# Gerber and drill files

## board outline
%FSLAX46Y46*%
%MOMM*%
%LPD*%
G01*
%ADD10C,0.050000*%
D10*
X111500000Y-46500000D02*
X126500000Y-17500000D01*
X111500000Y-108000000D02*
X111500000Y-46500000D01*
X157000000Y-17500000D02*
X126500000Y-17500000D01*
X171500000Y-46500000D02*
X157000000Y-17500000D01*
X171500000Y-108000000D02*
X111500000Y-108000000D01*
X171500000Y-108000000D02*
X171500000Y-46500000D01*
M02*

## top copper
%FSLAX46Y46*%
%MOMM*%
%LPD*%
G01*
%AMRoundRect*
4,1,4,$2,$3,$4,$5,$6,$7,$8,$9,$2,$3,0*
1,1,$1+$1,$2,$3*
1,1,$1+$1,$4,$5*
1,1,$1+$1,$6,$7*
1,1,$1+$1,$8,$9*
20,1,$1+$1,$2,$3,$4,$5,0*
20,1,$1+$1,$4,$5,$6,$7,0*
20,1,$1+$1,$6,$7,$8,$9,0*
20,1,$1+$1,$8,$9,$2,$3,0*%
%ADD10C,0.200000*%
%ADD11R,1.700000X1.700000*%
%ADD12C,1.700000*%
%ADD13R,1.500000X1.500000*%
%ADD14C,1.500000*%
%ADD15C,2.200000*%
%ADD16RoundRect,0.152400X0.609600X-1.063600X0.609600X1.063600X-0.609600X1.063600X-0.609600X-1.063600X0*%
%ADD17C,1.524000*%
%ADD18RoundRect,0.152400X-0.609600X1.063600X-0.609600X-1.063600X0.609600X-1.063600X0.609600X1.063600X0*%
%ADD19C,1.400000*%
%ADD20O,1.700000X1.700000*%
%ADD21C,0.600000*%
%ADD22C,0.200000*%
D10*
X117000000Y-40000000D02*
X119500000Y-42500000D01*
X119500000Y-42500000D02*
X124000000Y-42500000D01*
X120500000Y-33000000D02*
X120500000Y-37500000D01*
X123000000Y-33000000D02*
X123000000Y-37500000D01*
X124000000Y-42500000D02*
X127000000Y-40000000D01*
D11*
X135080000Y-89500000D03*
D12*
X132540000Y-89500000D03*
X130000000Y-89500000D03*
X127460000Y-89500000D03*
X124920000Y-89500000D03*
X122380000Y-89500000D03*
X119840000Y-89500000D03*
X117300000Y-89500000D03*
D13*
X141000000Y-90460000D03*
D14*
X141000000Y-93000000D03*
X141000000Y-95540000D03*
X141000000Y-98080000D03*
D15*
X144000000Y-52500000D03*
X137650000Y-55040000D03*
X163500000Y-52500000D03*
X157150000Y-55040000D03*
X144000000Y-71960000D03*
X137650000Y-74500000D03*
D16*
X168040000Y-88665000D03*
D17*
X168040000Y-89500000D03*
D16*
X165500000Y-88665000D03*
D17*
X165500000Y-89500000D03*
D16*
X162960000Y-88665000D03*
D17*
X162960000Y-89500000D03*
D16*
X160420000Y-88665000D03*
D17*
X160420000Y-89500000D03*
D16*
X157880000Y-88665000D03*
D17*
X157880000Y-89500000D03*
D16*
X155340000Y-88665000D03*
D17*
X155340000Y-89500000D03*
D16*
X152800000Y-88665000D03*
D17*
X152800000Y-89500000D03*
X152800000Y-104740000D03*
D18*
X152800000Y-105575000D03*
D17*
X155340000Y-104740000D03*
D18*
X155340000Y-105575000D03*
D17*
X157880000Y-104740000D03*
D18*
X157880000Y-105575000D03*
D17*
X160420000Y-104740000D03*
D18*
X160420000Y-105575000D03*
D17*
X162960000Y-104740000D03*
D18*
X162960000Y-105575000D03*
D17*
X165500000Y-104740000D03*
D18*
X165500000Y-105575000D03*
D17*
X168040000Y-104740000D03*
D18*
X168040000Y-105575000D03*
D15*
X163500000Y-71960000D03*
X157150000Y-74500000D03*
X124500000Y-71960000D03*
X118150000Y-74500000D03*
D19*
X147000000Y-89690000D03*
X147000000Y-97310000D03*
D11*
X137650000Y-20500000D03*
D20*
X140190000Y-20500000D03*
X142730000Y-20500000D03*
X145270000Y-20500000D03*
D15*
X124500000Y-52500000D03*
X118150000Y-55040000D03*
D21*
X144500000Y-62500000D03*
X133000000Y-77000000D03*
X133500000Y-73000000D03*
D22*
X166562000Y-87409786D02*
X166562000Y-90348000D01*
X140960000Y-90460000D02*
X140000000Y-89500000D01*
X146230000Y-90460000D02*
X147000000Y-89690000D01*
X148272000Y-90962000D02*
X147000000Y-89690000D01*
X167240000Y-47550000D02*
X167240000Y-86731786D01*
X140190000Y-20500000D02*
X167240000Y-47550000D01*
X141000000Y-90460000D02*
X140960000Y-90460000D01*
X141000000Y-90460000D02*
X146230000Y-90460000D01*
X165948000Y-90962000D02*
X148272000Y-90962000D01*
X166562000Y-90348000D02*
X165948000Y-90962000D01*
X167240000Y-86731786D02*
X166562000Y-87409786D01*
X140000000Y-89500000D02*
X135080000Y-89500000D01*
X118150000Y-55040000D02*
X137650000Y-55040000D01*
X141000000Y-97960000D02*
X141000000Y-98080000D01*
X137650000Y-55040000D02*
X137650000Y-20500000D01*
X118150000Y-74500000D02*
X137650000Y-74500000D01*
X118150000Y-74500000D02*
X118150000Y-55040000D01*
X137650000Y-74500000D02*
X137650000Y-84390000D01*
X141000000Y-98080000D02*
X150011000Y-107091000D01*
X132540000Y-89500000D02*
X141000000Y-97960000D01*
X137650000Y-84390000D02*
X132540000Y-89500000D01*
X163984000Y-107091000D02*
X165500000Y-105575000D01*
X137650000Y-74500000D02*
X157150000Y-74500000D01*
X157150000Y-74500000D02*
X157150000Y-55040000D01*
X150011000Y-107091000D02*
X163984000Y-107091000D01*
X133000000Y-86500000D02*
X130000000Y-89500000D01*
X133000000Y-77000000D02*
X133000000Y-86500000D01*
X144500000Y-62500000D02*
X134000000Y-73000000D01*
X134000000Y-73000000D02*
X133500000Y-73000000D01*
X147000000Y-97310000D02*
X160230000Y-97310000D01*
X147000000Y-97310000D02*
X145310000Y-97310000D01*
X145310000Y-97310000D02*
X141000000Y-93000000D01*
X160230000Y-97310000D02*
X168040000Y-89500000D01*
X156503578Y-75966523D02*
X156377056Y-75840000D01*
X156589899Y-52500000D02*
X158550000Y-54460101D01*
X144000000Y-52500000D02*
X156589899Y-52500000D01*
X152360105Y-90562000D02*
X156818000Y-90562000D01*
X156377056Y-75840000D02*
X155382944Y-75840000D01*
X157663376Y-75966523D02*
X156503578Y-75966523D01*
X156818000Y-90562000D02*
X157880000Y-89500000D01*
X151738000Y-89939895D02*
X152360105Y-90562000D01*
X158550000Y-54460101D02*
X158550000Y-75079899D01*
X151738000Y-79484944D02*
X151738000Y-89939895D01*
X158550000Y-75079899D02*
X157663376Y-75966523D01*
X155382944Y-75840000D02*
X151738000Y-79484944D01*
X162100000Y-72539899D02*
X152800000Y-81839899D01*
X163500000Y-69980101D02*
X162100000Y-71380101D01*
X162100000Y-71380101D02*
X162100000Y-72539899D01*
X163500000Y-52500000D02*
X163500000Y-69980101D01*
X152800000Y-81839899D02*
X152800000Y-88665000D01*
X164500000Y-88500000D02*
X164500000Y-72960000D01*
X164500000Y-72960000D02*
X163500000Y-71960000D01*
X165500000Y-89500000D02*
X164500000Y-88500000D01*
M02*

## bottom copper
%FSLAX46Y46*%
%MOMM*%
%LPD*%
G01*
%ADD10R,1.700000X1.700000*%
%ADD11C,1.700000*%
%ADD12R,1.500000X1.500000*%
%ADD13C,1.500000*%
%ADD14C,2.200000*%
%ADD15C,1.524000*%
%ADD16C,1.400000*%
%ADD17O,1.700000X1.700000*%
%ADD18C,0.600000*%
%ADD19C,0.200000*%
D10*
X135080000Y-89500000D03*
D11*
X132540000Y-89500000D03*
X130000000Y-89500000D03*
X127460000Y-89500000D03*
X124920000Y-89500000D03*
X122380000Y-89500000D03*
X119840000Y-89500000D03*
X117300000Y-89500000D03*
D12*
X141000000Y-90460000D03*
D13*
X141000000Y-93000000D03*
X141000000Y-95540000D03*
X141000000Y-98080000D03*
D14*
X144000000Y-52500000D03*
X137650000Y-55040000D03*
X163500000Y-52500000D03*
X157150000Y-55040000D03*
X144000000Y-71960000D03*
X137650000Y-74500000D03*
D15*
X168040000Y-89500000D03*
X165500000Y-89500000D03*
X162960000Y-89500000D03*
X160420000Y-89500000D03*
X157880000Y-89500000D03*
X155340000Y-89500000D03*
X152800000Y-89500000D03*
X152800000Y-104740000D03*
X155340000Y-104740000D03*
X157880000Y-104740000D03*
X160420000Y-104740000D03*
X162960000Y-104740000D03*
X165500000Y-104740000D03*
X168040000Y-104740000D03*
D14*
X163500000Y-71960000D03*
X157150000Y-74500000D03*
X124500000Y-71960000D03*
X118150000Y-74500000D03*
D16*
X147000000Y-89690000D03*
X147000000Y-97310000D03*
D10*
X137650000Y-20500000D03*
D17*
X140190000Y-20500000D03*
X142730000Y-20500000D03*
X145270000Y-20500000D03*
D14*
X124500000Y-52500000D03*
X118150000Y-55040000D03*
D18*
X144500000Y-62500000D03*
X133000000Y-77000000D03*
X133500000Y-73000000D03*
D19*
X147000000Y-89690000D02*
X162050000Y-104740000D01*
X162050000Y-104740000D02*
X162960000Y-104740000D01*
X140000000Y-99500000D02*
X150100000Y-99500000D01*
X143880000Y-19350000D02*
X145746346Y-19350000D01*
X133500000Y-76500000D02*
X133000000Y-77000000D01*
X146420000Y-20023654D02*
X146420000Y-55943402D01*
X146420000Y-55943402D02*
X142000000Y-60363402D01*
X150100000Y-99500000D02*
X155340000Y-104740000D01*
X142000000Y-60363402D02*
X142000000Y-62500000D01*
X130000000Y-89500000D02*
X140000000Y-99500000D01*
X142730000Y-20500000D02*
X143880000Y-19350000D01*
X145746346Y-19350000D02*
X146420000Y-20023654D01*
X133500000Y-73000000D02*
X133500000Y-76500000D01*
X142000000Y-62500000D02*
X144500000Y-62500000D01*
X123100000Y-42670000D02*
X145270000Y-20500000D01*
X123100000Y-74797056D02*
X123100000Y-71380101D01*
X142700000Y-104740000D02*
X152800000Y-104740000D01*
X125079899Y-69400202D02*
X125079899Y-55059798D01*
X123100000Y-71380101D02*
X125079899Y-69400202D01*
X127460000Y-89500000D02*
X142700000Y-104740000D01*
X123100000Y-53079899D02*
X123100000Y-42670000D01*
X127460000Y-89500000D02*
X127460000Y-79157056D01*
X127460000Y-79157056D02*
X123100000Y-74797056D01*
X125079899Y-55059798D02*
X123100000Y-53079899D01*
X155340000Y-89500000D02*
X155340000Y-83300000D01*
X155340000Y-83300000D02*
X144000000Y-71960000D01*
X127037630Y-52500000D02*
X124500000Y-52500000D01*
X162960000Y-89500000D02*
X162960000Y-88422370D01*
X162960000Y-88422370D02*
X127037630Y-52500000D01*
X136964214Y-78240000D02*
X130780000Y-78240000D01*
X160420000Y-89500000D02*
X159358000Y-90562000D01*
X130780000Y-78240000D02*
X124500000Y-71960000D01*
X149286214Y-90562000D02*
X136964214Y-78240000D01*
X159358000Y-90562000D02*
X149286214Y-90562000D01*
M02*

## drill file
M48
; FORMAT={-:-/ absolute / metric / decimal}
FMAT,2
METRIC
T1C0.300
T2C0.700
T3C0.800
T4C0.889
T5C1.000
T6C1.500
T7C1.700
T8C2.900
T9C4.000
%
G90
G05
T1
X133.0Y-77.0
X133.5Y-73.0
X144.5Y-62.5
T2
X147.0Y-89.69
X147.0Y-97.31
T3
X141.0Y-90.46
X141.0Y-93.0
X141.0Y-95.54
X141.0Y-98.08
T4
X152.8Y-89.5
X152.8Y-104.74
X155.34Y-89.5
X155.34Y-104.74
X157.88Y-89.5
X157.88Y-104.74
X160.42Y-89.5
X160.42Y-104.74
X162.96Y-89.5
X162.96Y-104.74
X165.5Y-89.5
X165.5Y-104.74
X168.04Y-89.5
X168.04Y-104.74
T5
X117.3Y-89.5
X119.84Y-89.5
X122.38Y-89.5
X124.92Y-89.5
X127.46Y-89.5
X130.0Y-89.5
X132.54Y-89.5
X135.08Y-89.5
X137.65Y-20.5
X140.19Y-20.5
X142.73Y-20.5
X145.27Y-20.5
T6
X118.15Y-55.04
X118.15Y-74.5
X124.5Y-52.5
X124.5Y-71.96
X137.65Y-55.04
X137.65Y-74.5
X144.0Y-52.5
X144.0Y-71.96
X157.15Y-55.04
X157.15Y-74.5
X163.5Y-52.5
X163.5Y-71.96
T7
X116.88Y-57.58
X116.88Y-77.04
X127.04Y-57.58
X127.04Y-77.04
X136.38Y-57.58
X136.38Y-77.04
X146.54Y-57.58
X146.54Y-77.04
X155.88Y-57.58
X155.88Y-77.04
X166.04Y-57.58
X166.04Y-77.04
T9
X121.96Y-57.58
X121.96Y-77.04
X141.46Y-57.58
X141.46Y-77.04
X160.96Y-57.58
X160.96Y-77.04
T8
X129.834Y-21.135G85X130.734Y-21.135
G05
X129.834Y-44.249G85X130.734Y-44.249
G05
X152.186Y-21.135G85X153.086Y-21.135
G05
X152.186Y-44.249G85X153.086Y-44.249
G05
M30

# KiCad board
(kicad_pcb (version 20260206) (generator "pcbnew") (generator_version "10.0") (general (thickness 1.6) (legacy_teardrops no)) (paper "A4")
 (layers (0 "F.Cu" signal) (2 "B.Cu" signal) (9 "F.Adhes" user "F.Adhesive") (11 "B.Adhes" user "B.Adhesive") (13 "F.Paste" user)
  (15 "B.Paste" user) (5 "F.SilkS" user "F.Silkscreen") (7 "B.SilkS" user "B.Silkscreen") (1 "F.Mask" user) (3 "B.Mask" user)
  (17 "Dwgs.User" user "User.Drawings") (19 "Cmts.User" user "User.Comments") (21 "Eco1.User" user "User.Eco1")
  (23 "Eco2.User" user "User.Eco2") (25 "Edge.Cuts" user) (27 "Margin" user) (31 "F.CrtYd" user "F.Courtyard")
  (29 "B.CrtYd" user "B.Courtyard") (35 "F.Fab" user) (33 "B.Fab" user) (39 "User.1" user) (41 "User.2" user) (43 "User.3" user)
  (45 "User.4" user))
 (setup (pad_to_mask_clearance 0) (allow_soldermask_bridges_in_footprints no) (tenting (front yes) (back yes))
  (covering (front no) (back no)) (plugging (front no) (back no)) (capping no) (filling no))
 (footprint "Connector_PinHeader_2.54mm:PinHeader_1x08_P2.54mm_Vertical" (layer "F.Cu") (at 135.08 89.5 -90)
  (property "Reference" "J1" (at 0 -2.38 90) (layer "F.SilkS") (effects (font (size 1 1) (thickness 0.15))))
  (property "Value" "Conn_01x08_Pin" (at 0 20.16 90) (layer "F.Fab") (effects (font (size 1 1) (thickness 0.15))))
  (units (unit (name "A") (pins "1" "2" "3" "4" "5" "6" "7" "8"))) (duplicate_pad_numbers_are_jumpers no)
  (pad "1" thru_hole rect (at 0 0 270) (size 1.7 1.7) (drill 1) (layers "*.Cu" "*.Mask") (remove_unused_layers no) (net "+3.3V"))
  (pad "2" thru_hole circle (at 0 2.54 270) (size 1.7 1.7) (drill 1) (layers "*.Cu" "*.Mask") (remove_unused_layers no) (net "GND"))
  (pad "3" thru_hole circle (at 0 5.08 270) (size 1.7 1.7) (drill 1) (layers "*.Cu" "*.Mask") (remove_unused_layers no) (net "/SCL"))
  (pad "4" thru_hole circle (at 0 7.62 270) (size 1.7 1.7) (drill 1) (layers "*.Cu" "*.Mask") (remove_unused_layers no) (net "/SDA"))
  (pad "5" thru_hole circle (at 0 10.16 270) (size 1.7 1.7) (drill 1) (layers "*.Cu" "*.Mask") (remove_unused_layers no)
   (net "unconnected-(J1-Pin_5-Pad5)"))
  (pad "6" thru_hole circle (at 0 12.7 270) (size 1.7 1.7) (drill 1) (layers "*.Cu" "*.Mask") (remove_unused_layers no)
   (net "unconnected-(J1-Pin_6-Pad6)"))
  (pad "7" thru_hole circle (at 0 15.24 270) (size 1.7 1.7) (drill 1) (layers "*.Cu" "*.Mask") (remove_unused_layers no)
   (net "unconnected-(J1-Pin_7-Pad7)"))
  (pad "8" thru_hole circle (at 0 17.78 270) (size 1.7 1.7) (drill 1) (layers "*.Cu" "*.Mask") (remove_unused_layers no)
   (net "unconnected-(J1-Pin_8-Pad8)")))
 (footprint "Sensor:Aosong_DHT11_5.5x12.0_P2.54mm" (layer "F.Cu") (at 141 90.46)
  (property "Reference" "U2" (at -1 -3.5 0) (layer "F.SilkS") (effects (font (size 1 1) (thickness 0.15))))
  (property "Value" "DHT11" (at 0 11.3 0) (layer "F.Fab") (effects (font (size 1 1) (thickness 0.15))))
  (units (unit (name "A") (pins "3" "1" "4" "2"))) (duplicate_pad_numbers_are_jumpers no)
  (pad "1" thru_hole rect (at 0 0) (size 1.5 1.5) (drill 0.8) (layers "*.Cu" "*.Mask") (remove_unused_layers no) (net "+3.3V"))
  (pad "2" thru_hole circle (at 0 2.54) (size 1.5 1.5) (drill 0.8) (layers "*.Cu" "*.Mask") (remove_unused_layers no) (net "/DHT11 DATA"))
  (pad "3" thru_hole circle (at 0 5.08) (size 1.5 1.5) (drill 0.8) (layers "*.Cu" "*.Mask") (remove_unused_layers no)
   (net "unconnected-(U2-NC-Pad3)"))
  (pad "4" thru_hole circle (at 0 7.62) (size 1.5 1.5) (drill 0.8) (layers "*.Cu" "*.Mask") (remove_unused_layers no) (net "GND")))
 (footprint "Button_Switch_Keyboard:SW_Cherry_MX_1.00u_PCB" (layer "F.Cu") (at 144 52.5)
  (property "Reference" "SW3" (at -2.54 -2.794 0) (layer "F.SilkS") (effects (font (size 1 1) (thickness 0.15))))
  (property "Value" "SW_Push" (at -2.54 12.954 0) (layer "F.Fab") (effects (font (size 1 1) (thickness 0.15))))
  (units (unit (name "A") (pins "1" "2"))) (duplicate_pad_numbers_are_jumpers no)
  (pad "" np_thru_hole circle (at -7.62 5.08) (size 1.7 1.7) (drill 1.7) (layers "*.Cu" "*.Mask"))
  (pad "" np_thru_hole circle (at -2.54 5.08) (size 4 4) (drill 4) (layers "*.Cu" "*.Mask"))
  (pad "" np_thru_hole circle (at 2.54 5.08) (size 1.7 1.7) (drill 1.7) (layers "*.Cu" "*.Mask"))
  (pad "1" thru_hole circle (at 0 0) (size 2.2 2.2) (drill 1.5) (layers "*.Cu" "*.Mask") (remove_unused_layers no) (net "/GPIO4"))
  (pad "2" thru_hole circle (at -6.35 2.54) (size 2.2 2.2) (drill 1.5) (layers "*.Cu" "*.Mask") (remove_unused_layers no) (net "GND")))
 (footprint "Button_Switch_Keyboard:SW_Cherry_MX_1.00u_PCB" (layer "F.Cu") (at 163.5 52.5)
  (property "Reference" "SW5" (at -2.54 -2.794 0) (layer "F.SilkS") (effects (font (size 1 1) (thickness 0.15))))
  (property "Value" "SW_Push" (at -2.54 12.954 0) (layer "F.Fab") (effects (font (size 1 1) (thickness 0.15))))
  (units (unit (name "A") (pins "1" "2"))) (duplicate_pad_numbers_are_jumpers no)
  (pad "" np_thru_hole circle (at -7.62 5.08) (size 1.7 1.7) (drill 1.7) (layers "*.Cu" "*.Mask"))
  (pad "" np_thru_hole circle (at -2.54 5.08) (size 4 4) (drill 4) (layers "*.Cu" "*.Mask"))
  (pad "" np_thru_hole circle (at 2.54 5.08) (size 1.7 1.7) (drill 1.7) (layers "*.Cu" "*.Mask"))
  (pad "1" thru_hole circle (at 0 0) (size 2.2 2.2) (drill 1.5) (layers "*.Cu" "*.Mask") (remove_unused_layers no) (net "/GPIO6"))
  (pad "2" thru_hole circle (at -6.35 2.54) (size 2.2 2.2) (drill 1.5) (layers "*.Cu" "*.Mask") (remove_unused_layers no) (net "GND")))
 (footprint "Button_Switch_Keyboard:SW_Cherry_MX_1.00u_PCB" (layer "F.Cu") (at 144 71.96)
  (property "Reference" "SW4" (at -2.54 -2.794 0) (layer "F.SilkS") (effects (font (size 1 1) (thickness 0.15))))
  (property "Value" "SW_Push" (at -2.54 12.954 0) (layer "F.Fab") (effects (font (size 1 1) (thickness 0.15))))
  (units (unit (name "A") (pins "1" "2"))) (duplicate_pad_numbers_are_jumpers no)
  (pad "" np_thru_hole circle (at -7.62 5.08) (size 1.7 1.7) (drill 1.7) (layers "*.Cu" "*.Mask"))
  (pad "" np_thru_hole circle (at -2.54 5.08) (size 4 4) (drill 4) (layers "*.Cu" "*.Mask"))
  (pad "" np_thru_hole circle (at 2.54 5.08) (size 1.7 1.7) (drill 1.7) (layers "*.Cu" "*.Mask"))
  (pad "1" thru_hole circle (at 0 0) (size 2.2 2.2) (drill 1.5) (layers "*.Cu" "*.Mask") (remove_unused_layers no) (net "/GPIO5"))
  (pad "2" thru_hole circle (at -6.35 2.54) (size 2.2 2.2) (drill 1.5) (layers "*.Cu" "*.Mask") (remove_unused_layers no) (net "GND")))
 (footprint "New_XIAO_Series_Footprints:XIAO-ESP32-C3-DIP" (layer "F.Cu") (at 160.42 97.12)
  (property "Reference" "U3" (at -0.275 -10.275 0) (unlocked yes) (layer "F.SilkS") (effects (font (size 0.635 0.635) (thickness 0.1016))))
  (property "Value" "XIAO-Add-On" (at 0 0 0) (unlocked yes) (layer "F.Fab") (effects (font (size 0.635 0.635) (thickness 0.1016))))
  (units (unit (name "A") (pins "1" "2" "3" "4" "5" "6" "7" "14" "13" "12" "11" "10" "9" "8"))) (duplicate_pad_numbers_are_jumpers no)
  (pad "1" smd roundrect (at 7.62 -8.455 90) (size 2.432 1.524) (layers "F.Cu" "F.Mask") (roundrect_rratio 0.1) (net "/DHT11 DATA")
   (thermal_bridge_angle 45))
  (pad "1" thru_hole circle (at 7.62 -7.62 90) (size 1.524 1.524) (drill 0.889) (layers "*.Cu" "*.Mask") (remove_unused_layers no)
   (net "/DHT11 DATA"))
  (pad "2" smd roundrect (at 5.08 -8.455 90) (size 2.432 1.524) (layers "F.Cu" "F.Mask") (roundrect_rratio 0.1) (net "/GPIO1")
   (thermal_bridge_angle 45))
  (pad "2" thru_hole circle (at 5.08 -7.62 90) (size 1.524 1.524) (drill 0.889) (layers "*.Cu" "*.Mask") (remove_unused_layers no)
   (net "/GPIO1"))
  (pad "3" smd roundrect (at 2.54 -8.455 90) (size 2.432 1.524) (layers "F.Cu" "F.Mask") (roundrect_rratio 0.1) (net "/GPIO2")
   (thermal_bridge_angle 45))
  (pad "3" thru_hole circle (at 2.54 -7.62 90) (size 1.524 1.524) (drill 0.889) (layers "*.Cu" "*.Mask") (remove_unused_layers no)
   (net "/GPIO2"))
  (pad "4" smd roundrect (at 0 -8.455 90) (size 2.432 1.524) (layers "F.Cu" "F.Mask") (roundrect_rratio 0.1) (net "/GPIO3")
   (thermal_bridge_angle 45))
  (pad "4" thru_hole circle (at 0 -7.62 90) (size 1.524 1.524) (drill 0.889) (layers "*.Cu" "*.Mask") (remove_unused_layers no)
   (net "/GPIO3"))
  (pad "5" smd roundrect (at -2.54 -8.455 90) (size 2.432 1.524) (layers "F.Cu" "F.Mask") (roundrect_rratio 0.1) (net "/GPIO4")
   (thermal_bridge_angle 45))
  (pad "5" thru_hole circle (at -2.54 -7.62 90) (size 1.524 1.524) (drill 0.889) (layers "*.Cu" "*.Mask") (remove_unused_layers no)
   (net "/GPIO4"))
  (pad "6" smd roundrect (at -5.08 -8.455 90) (size 2.432 1.524) (layers "F.Cu" "F.Mask") (roundrect_rratio 0.1) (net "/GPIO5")
   (thermal_bridge_angle 45))
  (pad "6" thru_hole circle (at -5.08 -7.62 90) (size 1.524 1.524) (drill 0.889) (layers "*.Cu" "*.Mask") (remove_unused_layers no)
   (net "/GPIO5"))
  (pad "7" smd roundrect (at -7.62 -8.455 90) (size 2.432 1.524) (layers "F.Cu" "F.Mask") (roundrect_rratio 0.1) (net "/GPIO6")
   (thermal_bridge_angle 45))
  (pad "7" thru_hole circle (at -7.62 -7.62 90) (size 1.524 1.524) (drill 0.889) (layers "*.Cu" "*.Mask") (remove_unused_layers no)
   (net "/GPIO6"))
  (pad "8" thru_hole circle (at -7.62 7.62 270) (size 1.524 1.524) (drill 0.889) (layers "*.Cu" "*.Mask") (remove_unused_layers no)
   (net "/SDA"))
  (pad "8" smd roundrect (at -7.62 8.455 270) (size 2.432 1.524) (layers "F.Cu" "F.Mask") (roundrect_rratio 0.1) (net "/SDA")
   (thermal_bridge_angle 45))
  (pad "9" thru_hole circle (at -5.08 7.62 270) (size 1.524 1.524) (drill 0.889) (layers "*.Cu" "*.Mask") (remove_unused_layers no)
   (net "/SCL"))
  (pad "9" smd roundrect (at -5.08 8.455 270) (size 2.432 1.524) (layers "F.Cu" "F.Mask") (roundrect_rratio 0.1) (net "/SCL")
   (thermal_bridge_angle 45))
  (pad "10" thru_hole circle (at -2.54 7.62 270) (size 1.524 1.524) (drill 0.889) (layers "*.Cu" "*.Mask") (remove_unused_layers no)
   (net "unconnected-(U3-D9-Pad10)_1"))
  (pad "10" smd roundrect (at -2.54 8.455 270) (size 2.432 1.524) (layers "F.Cu" "F.Mask") (roundrect_rratio 0.1)
   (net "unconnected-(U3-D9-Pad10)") (thermal_bridge_angle 45))
  (pad "11" thru_hole circle (at 0 7.62 270) (size 1.524 1.524) (drill 0.889) (layers "*.Cu" "*.Mask") (remove_unused_layers no)
   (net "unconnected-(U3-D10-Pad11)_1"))
  (pad "11" smd roundrect (at 0 8.455 270) (size 2.432 1.524) (layers "F.Cu" "F.Mask") (roundrect_rratio 0.1)
   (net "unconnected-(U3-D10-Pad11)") (thermal_bridge_angle 45))
  (pad "12" thru_hole circle (at 2.54 7.62 270) (size 1.524 1.524) (drill 0.889) (layers "*.Cu" "*.Mask") (remove_unused_layers no)
   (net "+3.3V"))
  (pad "12" smd roundrect (at 2.54 8.455 270) (size 2.432 1.524) (layers "F.Cu" "F.Mask") (roundrect_rratio 0.1) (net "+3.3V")
   (thermal_bridge_angle 45))
  (pad "13" thru_hole circle (at 5.08 7.62 270) (size 1.524 1.524) (drill 0.889) (layers "*.Cu" "*.Mask") (remove_unused_layers no)
   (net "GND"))
  (pad "13" smd roundrect (at 5.08 8.455 270) (size 2.432 1.524) (layers "F.Cu" "F.Mask") (roundrect_rratio 0.1) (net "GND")
   (thermal_bridge_angle 45))
  (pad "14" thru_hole circle (at 7.62 7.62 270) (size 1.524 1.524) (drill 0.889) (layers "*.Cu" "*.Mask") (remove_unused_layers no)
   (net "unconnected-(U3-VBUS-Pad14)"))
  (pad "14" smd roundrect (at 7.62 8.455 270) (size 2.432 1.524) (layers "F.Cu" "F.Mask") (roundrect_rratio 0.1)
   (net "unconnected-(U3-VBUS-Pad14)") (thermal_bridge_angle 45)))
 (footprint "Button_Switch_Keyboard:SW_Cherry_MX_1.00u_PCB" (layer "F.Cu") (at 163.5 71.96)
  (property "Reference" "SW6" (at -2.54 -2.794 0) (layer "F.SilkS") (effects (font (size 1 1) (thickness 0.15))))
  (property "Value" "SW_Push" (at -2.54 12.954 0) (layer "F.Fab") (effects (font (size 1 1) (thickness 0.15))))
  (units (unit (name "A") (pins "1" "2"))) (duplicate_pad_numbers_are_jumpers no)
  (pad "" np_thru_hole circle (at -7.62 5.08) (size 1.7 1.7) (drill 1.7) (layers "*.Cu" "*.Mask"))
  (pad "" np_thru_hole circle (at -2.54 5.08) (size 4 4) (drill 4) (layers "*.Cu" "*.Mask"))
  (pad "" np_thru_hole circle (at 2.54 5.08) (size 1.7 1.7) (drill 1.7) (layers "*.Cu" "*.Mask"))
  (pad "1" thru_hole circle (at 0 0) (size 2.2 2.2) (drill 1.5) (layers "*.Cu" "*.Mask") (remove_unused_layers no) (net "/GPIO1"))
  (pad "2" thru_hole circle (at -6.35 2.54) (size 2.2 2.2) (drill 1.5) (layers "*.Cu" "*.Mask") (remove_unused_layers no) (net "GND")))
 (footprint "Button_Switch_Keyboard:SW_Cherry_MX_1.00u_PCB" (layer "F.Cu") (at 124.5 71.96)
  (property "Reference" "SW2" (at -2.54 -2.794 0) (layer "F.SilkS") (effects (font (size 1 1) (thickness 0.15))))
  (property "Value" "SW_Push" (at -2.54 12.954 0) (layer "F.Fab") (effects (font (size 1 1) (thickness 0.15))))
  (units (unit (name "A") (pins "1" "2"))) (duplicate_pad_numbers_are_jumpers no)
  (pad "" np_thru_hole circle (at -7.62 5.08) (size 1.7 1.7) (drill 1.7) (layers "*.Cu" "*.Mask"))
  (pad "" np_thru_hole circle (at -2.54 5.08) (size 4 4) (drill 4) (layers "*.Cu" "*.Mask"))
  (pad "" np_thru_hole circle (at 2.54 5.08) (size 1.7 1.7) (drill 1.7) (layers "*.Cu" "*.Mask"))
  (pad "1" thru_hole circle (at 0 0) (size 2.2 2.2) (drill 1.5) (layers "*.Cu" "*.Mask") (remove_unused_layers no) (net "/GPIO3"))
  (pad "2" thru_hole circle (at -6.35 2.54) (size 2.2 2.2) (drill 1.5) (layers "*.Cu" "*.Mask") (remove_unused_layers no) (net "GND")))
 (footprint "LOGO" (layer "F.Cu") (at 161.5 39.5)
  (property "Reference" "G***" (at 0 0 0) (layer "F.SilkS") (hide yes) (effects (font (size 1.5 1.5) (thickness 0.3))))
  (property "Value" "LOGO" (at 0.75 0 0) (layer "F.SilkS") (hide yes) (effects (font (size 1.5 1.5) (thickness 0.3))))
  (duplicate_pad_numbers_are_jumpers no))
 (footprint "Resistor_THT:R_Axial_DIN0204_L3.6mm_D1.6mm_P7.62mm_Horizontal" (layer "F.Cu") (at 147 89.69 -90)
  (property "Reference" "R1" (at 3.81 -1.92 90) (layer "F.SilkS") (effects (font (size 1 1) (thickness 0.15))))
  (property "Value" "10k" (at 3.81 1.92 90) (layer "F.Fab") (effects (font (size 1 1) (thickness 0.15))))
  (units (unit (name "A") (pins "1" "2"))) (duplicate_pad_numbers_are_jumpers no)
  (pad "1" thru_hole circle (at 0 0 270) (size 1.4 1.4) (drill 0.7) (layers "*.Cu" "*.Mask") (remove_unused_layers no) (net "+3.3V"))
  (pad "2" thru_hole circle (at 7.62 0 270) (size 1.4 1.4) (drill 0.7) (layers "*.Cu" "*.Mask") (remove_unused_layers no)
   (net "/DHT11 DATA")))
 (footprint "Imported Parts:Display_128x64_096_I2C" (layer "F.Cu") (at 141.46 20.5)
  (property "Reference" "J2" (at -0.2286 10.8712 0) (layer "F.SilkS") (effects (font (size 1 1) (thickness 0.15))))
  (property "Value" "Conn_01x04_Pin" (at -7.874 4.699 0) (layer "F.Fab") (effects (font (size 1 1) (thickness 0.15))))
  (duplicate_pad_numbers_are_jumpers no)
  (pad "" np_thru_hole oval (at -11.176 0.635) (size 3.8 2.9) (drill oval 3.8 2.9) (layers "*.Cu" "*.Mask"))
  (pad "" np_thru_hole oval (at -11.176 23.749) (size 3.8 2.9) (drill oval 3.8 2.9) (layers "*.Cu" "*.Mask"))
  (pad "" np_thru_hole oval (at 11.176 0.635) (size 3.8 2.9) (drill oval 3.8 2.9) (layers "*.Cu" "*.Mask"))
  (pad "" np_thru_hole oval (at 11.176 23.749) (size 3.8 2.9) (drill oval 3.8 2.9) (layers "*.Cu" "*.Mask"))
  (pad "1" thru_hole rect (at -3.81 0 90) (size 1.7 1.7) (drill 1) (layers "*.Cu" "*.Mask") (remove_unused_layers no) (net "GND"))
  (pad "2" thru_hole oval (at -1.27 0 90) (size 1.7 1.7) (drill 1) (layers "*.Cu" "*.Mask") (remove_unused_layers no) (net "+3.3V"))
  (pad "3" thru_hole oval (at 1.27 0 90) (size 1.7 1.7) (drill 1) (layers "*.Cu" "*.Mask") (remove_unused_layers no) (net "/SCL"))
  (pad "4" thru_hole oval (at 3.81 0 90) (size 1.7 1.7) (drill 1) (layers "*.Cu" "*.Mask") (remove_unused_layers no) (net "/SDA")))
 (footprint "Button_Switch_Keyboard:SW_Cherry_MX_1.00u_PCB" (layer "F.Cu") (at 124.5 52.5)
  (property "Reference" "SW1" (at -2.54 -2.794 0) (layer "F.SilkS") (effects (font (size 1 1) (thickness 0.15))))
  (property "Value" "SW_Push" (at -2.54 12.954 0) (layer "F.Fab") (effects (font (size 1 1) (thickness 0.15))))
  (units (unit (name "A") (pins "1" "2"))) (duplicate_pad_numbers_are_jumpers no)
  (pad "" np_thru_hole circle (at -7.62 5.08) (size 1.7 1.7) (drill 1.7) (layers "*.Cu" "*.Mask"))
  (pad "" np_thru_hole circle (at -2.54 5.08) (size 4 4) (drill 4) (layers "*.Cu" "*.Mask"))
  (pad "" np_thru_hole circle (at 2.54 5.08) (size 1.7 1.7) (drill 1.7) (layers "*.Cu" "*.Mask"))
  (pad "1" thru_hole circle (at 0 0) (size 2.2 2.2) (drill 1.5) (layers "*.Cu" "*.Mask") (remove_unused_layers no) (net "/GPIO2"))
  (pad "2" thru_hole circle (at -6.35 2.54) (size 2.2 2.2) (drill 1.5) (layers "*.Cu" "*.Mask") (remove_unused_layers no) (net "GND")))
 (gr_line (start 117 40) (end 119.5 42.5) (stroke (width 0.2) (type default)) (layer "F.Cu"))
 (gr_line (start 119.5 42.5) (end 124 42.5) (stroke (width 0.2) (type default)) (layer "F.Cu"))
 (gr_line (start 120.5 33) (end 120.5 37.5) (stroke (width 0.2) (type default)) (layer "F.Cu"))
 (gr_line (start 123 33) (end 123 37.5) (stroke (width 0.2) (type default)) (layer "F.Cu"))
 (gr_line (start 124 42.5) (end 127 40) (stroke (width 0.2) (type default)) (layer "F.Cu"))
 (gr_line (start 111.5 46.5) (end 126.5 17.5) (stroke (width 0.05) (type default)) (layer "Edge.Cuts"))
 (gr_line (start 111.5 108) (end 111.5 46.5) (stroke (width 0.05) (type default)) (layer "Edge.Cuts"))
 (gr_line (start 157 17.5) (end 126.5 17.5) (stroke (width 0.05) (type default)) (layer "Edge.Cuts"))
 (gr_line (start 171.5 46.5) (end 157 17.5) (stroke (width 0.05) (type default)) (layer "Edge.Cuts"))
 (gr_line (start 171.5 108) (end 111.5 108) (stroke (width 0.05) (type default)) (layer "Edge.Cuts"))
 (gr_line (start 171.5 108) (end 171.5 46.5) (stroke (width 0.05) (type default)) (layer "Edge.Cuts"))
 (segment (start 166.562 87.409786) (end 166.562 90.348) (width 0.2) (layer "F.Cu") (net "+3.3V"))
 (segment (start 140.96 90.46) (end 140 89.5) (width 0.2) (layer "F.Cu") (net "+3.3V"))
 (segment (start 146.23 90.46) (end 147 89.69) (width 0.2) (layer "F.Cu") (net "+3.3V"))
 (segment (start 148.272 90.962) (end 147 89.69) (width 0.2) (layer "F.Cu") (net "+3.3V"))
 (segment (start 167.24 47.55) (end 167.24 86.731786) (width 0.2) (layer "F.Cu") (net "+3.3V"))
 (segment (start 140.19 20.5) (end 167.24 47.55) (width 0.2) (layer "F.Cu") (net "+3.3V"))
 (segment (start 141 90.46) (end 140.96 90.46) (width 0.2) (layer "F.Cu") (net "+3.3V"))
 (segment (start 141 90.46) (end 146.23 90.46) (width 0.2) (layer "F.Cu") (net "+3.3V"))
 (segment (start 165.948 90.962) (end 148.272 90.962) (width 0.2) (layer "F.Cu") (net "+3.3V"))
 (segment (start 166.562 90.348) (end 165.948 90.962) (width 0.2) (layer "F.Cu") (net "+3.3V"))
 (segment (start 167.24 86.731786) (end 166.562 87.409786) (width 0.2) (layer "F.Cu") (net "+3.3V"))
 (segment (start 140 89.5) (end 135.08 89.5) (width 0.2) (layer "F.Cu") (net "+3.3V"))
 (segment (start 147 89.69) (end 162.05 104.74) (width 0.2) (layer "B.Cu") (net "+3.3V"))
 (segment (start 162.05 104.74) (end 162.96 104.74) (width 0.2) (layer "B.Cu") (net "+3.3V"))
 (segment (start 118.15 55.04) (end 137.65 55.04) (width 0.2) (layer "F.Cu") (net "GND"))
 (segment (start 141 97.96) (end 141 98.08) (width 0.2) (layer "F.Cu") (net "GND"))
 (segment (start 137.65 55.04) (end 137.65 20.5) (width 0.2) (layer "F.Cu") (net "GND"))
 (segment (start 118.15 74.5) (end 137.65 74.5) (width 0.2) (layer "F.Cu") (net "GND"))
 (segment (start 118.15 74.5) (end 118.15 55.04) (width 0.2) (layer "F.Cu") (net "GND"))
 (segment (start 137.65 74.5) (end 137.65 84.39) (width 0.2) (layer "F.Cu") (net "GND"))
 (segment (start 141 98.08) (end 150.011 107.091) (width 0.2) (layer "F.Cu") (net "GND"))
 (segment (start 132.54 89.5) (end 141 97.96) (width 0.2) (layer "F.Cu") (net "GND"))
 (segment (start 137.65 84.39) (end 132.54 89.5) (width 0.2) (layer "F.Cu") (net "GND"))
 (segment (start 163.984 107.091) (end 165.5 105.575) (width 0.2) (layer "F.Cu") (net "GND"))
 (segment (start 137.65 74.5) (end 157.15 74.5) (width 0.2) (layer "F.Cu") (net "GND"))
 (segment (start 157.15 74.5) (end 157.15 55.04) (width 0.2) (layer "F.Cu") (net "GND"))
 (segment (start 150.011 107.091) (end 163.984 107.091) (width 0.2) (layer "F.Cu") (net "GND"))
 (segment (start 133 86.5) (end 130 89.5) (width 0.2) (layer "F.Cu") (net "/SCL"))
 (segment (start 133 77) (end 133 86.5) (width 0.2) (layer "F.Cu") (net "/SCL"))
 (segment (start 144.5 62.5) (end 134 73) (width 0.2) (layer "F.Cu") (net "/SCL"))
 (segment (start 134 73) (end 133.5 73) (width 0.2) (layer "F.Cu") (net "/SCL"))
 (via (at 144.5 62.5) (size 0.6) (drill 0.3) (layers "F.Cu" "B.Cu") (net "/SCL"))
 (via (at 133 77) (size 0.6) (drill 0.3) (layers "F.Cu" "B.Cu") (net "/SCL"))
 (via (at 133.5 73) (size 0.6) (drill 0.3) (layers "F.Cu" "B.Cu") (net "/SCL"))
 (segment (start 140 99.5) (end 150.1 99.5) (width 0.2) (layer "B.Cu") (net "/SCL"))
 (segment (start 143.88 19.35) (end 145.746346 19.35) (width 0.2) (layer "B.Cu") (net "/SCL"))
 (segment (start 133.5 76.5) (end 133 77) (width 0.2) (layer "B.Cu") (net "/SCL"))
 (segment (start 146.42 20.023654) (end 146.42 55.943402) (width 0.2) (layer "B.Cu") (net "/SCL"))
 (segment (start 146.42 55.943402) (end 142 60.363402) (width 0.2) (layer "B.Cu") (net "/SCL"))
 (segment (start 150.1 99.5) (end 155.34 104.74) (width 0.2) (layer "B.Cu") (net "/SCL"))
 (segment (start 142 60.363402) (end 142 62.5) (width 0.2) (layer "B.Cu") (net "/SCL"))
 (segment (start 130 89.5) (end 140 99.5) (width 0.2) (layer "B.Cu") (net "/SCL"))
 (segment (start 142.73 20.5) (end 143.88 19.35) (width 0.2) (layer "B.Cu") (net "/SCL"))
 (segment (start 145.746346 19.35) (end 146.42 20.023654) (width 0.2) (layer "B.Cu") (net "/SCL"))
 (segment (start 133.5 73) (end 133.5 76.5) (width 0.2) (layer "B.Cu") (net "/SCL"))
 (segment (start 142 62.5) (end 144.5 62.5) (width 0.2) (layer "B.Cu") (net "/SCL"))
 (segment (start 123.1 42.67) (end 145.27 20.5) (width 0.2) (layer "B.Cu") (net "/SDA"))
 (segment (start 123.1 74.797056) (end 123.1 71.380101) (width 0.2) (layer "B.Cu") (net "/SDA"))
 (segment (start 142.7 104.74) (end 152.8 104.74) (width 0.2) (layer "B.Cu") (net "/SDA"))
 (segment (start 125.079899 69.400202) (end 125.079899 55.059798) (width 0.2) (layer "B.Cu") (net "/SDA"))
 (segment (start 123.1 71.380101) (end 125.079899 69.400202) (width 0.2) (layer "B.Cu") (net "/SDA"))
 (segment (start 127.46 89.5) (end 142.7 104.74) (width 0.2) (layer "B.Cu") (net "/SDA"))
 (segment (start 123.1 53.079899) (end 123.1 42.67) (width 0.2) (layer "B.Cu") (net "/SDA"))
 (segment (start 127.46 89.5) (end 127.46 79.157056) (width 0.2) (layer "B.Cu") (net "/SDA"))
 (segment (start 127.46 79.157056) (end 123.1 74.797056) (width 0.2) (layer "B.Cu") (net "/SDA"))
 (segment (start 125.079899 55.059798) (end 123.1 53.079899) (width 0.2) (layer "B.Cu") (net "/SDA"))
 (segment (start 147 97.31) (end 160.23 97.31) (width 0.2) (layer "F.Cu") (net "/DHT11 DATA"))
 (segment (start 147 97.31) (end 145.31 97.31) (width 0.2) (layer "F.Cu") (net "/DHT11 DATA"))
 (segment (start 145.31 97.31) (end 141 93) (width 0.2) (layer "F.Cu") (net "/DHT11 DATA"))
 (segment (start 160.23 97.31) (end 168.04 89.5) (width 0.2) (layer "F.Cu") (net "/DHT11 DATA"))
 (segment (start 156.503578 75.966523) (end 156.377056 75.84) (width 0.2) (layer "F.Cu") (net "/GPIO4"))
 (segment (start 156.589899 52.5) (end 158.55 54.460101) (width 0.2) (layer "F.Cu") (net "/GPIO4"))
 (segment (start 144 52.5) (end 156.589899 52.5) (width 0.2) (layer "F.Cu") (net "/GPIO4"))
 (segment (start 152.360105 90.562) (end 156.818 90.562) (width 0.2) (layer "F.Cu") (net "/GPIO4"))
 (segment (start 156.377056 75.84) (end 155.382944 75.84) (width 0.2) (layer "F.Cu") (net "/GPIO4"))
 (segment (start 157.663376 75.966523) (end 156.503578 75.966523) (width 0.2) (layer "F.Cu") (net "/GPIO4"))
 (segment (start 156.818 90.562) (end 157.88 89.5) (width 0.2) (layer "F.Cu") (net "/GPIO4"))
 (segment (start 151.738 89.939895) (end 152.360105 90.562) (width 0.2) (layer "F.Cu") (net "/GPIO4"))
 (segment (start 158.55 54.460101) (end 158.55 75.079899) (width 0.2) (layer "F.Cu") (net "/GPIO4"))
 (segment (start 151.738 79.484944) (end 151.738 89.939895) (width 0.2) (layer "F.Cu") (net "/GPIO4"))
 (segment (start 158.55 75.079899) (end 157.663376 75.966523) (width 0.2) (layer "F.Cu") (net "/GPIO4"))
 (segment (start 155.382944 75.84) (end 151.738 79.484944) (width 0.2) (layer "F.Cu") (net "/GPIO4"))
 (segment (start 162.1 72.539899) (end 152.8 81.839899) (width 0.2) (layer "F.Cu") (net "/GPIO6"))
 (segment (start 163.5 69.980101) (end 162.1 71.380101) (width 0.2) (layer "F.Cu") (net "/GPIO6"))
 (segment (start 162.1 71.380101) (end 162.1 72.539899) (width 0.2) (layer "F.Cu") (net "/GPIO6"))
 (segment (start 163.5 52.5) (end 163.5 69.980101) (width 0.2) (layer "F.Cu") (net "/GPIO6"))
 (segment (start 152.8 81.839899) (end 152.8 88.665) (width 0.2) (layer "F.Cu") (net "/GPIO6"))
 (segment (start 155.34 89.5) (end 155.34 83.3) (width 0.2) (layer "B.Cu") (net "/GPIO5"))
 (segment (start 155.34 83.3) (end 144 71.96) (width 0.2) (layer "B.Cu") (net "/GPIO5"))
 (segment (start 164.5 88.5) (end 164.5 72.96) (width 0.2) (layer "F.Cu") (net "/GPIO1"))
 (segment (start 164.5 72.96) (end 163.5 71.96) (width 0.2) (layer "F.Cu") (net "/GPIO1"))
 (segment (start 165.5 89.5) (end 164.5 88.5) (width 0.2) (layer "F.Cu") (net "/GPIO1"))
 (segment (start 127.03763 52.5) (end 124.5 52.5) (width 0.2) (layer "B.Cu") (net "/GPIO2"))
 (segment (start 162.96 89.5) (end 162.96 88.42237) (width 0.2) (layer "B.Cu") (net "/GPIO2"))
 (segment (start 162.96 88.42237) (end 127.03763 52.5) (width 0.2) (layer "B.Cu") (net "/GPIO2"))
 (segment (start 136.964214 78.24) (end 130.78 78.24) (width 0.2) (layer "B.Cu") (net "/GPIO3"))
 (segment (start 160.42 89.5) (end 159.358 90.562) (width 0.2) (layer "B.Cu") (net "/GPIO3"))
 (segment (start 130.78 78.24) (end 124.5 71.96) (width 0.2) (layer "B.Cu") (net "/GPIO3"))
 (segment (start 149.286214 90.562) (end 136.964214 78.24) (width 0.2) (layer "B.Cu") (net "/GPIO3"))
 (segment (start 159.358 90.562) (end 149.286214 90.562) (width 0.2) (layer "B.Cu") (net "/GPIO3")))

